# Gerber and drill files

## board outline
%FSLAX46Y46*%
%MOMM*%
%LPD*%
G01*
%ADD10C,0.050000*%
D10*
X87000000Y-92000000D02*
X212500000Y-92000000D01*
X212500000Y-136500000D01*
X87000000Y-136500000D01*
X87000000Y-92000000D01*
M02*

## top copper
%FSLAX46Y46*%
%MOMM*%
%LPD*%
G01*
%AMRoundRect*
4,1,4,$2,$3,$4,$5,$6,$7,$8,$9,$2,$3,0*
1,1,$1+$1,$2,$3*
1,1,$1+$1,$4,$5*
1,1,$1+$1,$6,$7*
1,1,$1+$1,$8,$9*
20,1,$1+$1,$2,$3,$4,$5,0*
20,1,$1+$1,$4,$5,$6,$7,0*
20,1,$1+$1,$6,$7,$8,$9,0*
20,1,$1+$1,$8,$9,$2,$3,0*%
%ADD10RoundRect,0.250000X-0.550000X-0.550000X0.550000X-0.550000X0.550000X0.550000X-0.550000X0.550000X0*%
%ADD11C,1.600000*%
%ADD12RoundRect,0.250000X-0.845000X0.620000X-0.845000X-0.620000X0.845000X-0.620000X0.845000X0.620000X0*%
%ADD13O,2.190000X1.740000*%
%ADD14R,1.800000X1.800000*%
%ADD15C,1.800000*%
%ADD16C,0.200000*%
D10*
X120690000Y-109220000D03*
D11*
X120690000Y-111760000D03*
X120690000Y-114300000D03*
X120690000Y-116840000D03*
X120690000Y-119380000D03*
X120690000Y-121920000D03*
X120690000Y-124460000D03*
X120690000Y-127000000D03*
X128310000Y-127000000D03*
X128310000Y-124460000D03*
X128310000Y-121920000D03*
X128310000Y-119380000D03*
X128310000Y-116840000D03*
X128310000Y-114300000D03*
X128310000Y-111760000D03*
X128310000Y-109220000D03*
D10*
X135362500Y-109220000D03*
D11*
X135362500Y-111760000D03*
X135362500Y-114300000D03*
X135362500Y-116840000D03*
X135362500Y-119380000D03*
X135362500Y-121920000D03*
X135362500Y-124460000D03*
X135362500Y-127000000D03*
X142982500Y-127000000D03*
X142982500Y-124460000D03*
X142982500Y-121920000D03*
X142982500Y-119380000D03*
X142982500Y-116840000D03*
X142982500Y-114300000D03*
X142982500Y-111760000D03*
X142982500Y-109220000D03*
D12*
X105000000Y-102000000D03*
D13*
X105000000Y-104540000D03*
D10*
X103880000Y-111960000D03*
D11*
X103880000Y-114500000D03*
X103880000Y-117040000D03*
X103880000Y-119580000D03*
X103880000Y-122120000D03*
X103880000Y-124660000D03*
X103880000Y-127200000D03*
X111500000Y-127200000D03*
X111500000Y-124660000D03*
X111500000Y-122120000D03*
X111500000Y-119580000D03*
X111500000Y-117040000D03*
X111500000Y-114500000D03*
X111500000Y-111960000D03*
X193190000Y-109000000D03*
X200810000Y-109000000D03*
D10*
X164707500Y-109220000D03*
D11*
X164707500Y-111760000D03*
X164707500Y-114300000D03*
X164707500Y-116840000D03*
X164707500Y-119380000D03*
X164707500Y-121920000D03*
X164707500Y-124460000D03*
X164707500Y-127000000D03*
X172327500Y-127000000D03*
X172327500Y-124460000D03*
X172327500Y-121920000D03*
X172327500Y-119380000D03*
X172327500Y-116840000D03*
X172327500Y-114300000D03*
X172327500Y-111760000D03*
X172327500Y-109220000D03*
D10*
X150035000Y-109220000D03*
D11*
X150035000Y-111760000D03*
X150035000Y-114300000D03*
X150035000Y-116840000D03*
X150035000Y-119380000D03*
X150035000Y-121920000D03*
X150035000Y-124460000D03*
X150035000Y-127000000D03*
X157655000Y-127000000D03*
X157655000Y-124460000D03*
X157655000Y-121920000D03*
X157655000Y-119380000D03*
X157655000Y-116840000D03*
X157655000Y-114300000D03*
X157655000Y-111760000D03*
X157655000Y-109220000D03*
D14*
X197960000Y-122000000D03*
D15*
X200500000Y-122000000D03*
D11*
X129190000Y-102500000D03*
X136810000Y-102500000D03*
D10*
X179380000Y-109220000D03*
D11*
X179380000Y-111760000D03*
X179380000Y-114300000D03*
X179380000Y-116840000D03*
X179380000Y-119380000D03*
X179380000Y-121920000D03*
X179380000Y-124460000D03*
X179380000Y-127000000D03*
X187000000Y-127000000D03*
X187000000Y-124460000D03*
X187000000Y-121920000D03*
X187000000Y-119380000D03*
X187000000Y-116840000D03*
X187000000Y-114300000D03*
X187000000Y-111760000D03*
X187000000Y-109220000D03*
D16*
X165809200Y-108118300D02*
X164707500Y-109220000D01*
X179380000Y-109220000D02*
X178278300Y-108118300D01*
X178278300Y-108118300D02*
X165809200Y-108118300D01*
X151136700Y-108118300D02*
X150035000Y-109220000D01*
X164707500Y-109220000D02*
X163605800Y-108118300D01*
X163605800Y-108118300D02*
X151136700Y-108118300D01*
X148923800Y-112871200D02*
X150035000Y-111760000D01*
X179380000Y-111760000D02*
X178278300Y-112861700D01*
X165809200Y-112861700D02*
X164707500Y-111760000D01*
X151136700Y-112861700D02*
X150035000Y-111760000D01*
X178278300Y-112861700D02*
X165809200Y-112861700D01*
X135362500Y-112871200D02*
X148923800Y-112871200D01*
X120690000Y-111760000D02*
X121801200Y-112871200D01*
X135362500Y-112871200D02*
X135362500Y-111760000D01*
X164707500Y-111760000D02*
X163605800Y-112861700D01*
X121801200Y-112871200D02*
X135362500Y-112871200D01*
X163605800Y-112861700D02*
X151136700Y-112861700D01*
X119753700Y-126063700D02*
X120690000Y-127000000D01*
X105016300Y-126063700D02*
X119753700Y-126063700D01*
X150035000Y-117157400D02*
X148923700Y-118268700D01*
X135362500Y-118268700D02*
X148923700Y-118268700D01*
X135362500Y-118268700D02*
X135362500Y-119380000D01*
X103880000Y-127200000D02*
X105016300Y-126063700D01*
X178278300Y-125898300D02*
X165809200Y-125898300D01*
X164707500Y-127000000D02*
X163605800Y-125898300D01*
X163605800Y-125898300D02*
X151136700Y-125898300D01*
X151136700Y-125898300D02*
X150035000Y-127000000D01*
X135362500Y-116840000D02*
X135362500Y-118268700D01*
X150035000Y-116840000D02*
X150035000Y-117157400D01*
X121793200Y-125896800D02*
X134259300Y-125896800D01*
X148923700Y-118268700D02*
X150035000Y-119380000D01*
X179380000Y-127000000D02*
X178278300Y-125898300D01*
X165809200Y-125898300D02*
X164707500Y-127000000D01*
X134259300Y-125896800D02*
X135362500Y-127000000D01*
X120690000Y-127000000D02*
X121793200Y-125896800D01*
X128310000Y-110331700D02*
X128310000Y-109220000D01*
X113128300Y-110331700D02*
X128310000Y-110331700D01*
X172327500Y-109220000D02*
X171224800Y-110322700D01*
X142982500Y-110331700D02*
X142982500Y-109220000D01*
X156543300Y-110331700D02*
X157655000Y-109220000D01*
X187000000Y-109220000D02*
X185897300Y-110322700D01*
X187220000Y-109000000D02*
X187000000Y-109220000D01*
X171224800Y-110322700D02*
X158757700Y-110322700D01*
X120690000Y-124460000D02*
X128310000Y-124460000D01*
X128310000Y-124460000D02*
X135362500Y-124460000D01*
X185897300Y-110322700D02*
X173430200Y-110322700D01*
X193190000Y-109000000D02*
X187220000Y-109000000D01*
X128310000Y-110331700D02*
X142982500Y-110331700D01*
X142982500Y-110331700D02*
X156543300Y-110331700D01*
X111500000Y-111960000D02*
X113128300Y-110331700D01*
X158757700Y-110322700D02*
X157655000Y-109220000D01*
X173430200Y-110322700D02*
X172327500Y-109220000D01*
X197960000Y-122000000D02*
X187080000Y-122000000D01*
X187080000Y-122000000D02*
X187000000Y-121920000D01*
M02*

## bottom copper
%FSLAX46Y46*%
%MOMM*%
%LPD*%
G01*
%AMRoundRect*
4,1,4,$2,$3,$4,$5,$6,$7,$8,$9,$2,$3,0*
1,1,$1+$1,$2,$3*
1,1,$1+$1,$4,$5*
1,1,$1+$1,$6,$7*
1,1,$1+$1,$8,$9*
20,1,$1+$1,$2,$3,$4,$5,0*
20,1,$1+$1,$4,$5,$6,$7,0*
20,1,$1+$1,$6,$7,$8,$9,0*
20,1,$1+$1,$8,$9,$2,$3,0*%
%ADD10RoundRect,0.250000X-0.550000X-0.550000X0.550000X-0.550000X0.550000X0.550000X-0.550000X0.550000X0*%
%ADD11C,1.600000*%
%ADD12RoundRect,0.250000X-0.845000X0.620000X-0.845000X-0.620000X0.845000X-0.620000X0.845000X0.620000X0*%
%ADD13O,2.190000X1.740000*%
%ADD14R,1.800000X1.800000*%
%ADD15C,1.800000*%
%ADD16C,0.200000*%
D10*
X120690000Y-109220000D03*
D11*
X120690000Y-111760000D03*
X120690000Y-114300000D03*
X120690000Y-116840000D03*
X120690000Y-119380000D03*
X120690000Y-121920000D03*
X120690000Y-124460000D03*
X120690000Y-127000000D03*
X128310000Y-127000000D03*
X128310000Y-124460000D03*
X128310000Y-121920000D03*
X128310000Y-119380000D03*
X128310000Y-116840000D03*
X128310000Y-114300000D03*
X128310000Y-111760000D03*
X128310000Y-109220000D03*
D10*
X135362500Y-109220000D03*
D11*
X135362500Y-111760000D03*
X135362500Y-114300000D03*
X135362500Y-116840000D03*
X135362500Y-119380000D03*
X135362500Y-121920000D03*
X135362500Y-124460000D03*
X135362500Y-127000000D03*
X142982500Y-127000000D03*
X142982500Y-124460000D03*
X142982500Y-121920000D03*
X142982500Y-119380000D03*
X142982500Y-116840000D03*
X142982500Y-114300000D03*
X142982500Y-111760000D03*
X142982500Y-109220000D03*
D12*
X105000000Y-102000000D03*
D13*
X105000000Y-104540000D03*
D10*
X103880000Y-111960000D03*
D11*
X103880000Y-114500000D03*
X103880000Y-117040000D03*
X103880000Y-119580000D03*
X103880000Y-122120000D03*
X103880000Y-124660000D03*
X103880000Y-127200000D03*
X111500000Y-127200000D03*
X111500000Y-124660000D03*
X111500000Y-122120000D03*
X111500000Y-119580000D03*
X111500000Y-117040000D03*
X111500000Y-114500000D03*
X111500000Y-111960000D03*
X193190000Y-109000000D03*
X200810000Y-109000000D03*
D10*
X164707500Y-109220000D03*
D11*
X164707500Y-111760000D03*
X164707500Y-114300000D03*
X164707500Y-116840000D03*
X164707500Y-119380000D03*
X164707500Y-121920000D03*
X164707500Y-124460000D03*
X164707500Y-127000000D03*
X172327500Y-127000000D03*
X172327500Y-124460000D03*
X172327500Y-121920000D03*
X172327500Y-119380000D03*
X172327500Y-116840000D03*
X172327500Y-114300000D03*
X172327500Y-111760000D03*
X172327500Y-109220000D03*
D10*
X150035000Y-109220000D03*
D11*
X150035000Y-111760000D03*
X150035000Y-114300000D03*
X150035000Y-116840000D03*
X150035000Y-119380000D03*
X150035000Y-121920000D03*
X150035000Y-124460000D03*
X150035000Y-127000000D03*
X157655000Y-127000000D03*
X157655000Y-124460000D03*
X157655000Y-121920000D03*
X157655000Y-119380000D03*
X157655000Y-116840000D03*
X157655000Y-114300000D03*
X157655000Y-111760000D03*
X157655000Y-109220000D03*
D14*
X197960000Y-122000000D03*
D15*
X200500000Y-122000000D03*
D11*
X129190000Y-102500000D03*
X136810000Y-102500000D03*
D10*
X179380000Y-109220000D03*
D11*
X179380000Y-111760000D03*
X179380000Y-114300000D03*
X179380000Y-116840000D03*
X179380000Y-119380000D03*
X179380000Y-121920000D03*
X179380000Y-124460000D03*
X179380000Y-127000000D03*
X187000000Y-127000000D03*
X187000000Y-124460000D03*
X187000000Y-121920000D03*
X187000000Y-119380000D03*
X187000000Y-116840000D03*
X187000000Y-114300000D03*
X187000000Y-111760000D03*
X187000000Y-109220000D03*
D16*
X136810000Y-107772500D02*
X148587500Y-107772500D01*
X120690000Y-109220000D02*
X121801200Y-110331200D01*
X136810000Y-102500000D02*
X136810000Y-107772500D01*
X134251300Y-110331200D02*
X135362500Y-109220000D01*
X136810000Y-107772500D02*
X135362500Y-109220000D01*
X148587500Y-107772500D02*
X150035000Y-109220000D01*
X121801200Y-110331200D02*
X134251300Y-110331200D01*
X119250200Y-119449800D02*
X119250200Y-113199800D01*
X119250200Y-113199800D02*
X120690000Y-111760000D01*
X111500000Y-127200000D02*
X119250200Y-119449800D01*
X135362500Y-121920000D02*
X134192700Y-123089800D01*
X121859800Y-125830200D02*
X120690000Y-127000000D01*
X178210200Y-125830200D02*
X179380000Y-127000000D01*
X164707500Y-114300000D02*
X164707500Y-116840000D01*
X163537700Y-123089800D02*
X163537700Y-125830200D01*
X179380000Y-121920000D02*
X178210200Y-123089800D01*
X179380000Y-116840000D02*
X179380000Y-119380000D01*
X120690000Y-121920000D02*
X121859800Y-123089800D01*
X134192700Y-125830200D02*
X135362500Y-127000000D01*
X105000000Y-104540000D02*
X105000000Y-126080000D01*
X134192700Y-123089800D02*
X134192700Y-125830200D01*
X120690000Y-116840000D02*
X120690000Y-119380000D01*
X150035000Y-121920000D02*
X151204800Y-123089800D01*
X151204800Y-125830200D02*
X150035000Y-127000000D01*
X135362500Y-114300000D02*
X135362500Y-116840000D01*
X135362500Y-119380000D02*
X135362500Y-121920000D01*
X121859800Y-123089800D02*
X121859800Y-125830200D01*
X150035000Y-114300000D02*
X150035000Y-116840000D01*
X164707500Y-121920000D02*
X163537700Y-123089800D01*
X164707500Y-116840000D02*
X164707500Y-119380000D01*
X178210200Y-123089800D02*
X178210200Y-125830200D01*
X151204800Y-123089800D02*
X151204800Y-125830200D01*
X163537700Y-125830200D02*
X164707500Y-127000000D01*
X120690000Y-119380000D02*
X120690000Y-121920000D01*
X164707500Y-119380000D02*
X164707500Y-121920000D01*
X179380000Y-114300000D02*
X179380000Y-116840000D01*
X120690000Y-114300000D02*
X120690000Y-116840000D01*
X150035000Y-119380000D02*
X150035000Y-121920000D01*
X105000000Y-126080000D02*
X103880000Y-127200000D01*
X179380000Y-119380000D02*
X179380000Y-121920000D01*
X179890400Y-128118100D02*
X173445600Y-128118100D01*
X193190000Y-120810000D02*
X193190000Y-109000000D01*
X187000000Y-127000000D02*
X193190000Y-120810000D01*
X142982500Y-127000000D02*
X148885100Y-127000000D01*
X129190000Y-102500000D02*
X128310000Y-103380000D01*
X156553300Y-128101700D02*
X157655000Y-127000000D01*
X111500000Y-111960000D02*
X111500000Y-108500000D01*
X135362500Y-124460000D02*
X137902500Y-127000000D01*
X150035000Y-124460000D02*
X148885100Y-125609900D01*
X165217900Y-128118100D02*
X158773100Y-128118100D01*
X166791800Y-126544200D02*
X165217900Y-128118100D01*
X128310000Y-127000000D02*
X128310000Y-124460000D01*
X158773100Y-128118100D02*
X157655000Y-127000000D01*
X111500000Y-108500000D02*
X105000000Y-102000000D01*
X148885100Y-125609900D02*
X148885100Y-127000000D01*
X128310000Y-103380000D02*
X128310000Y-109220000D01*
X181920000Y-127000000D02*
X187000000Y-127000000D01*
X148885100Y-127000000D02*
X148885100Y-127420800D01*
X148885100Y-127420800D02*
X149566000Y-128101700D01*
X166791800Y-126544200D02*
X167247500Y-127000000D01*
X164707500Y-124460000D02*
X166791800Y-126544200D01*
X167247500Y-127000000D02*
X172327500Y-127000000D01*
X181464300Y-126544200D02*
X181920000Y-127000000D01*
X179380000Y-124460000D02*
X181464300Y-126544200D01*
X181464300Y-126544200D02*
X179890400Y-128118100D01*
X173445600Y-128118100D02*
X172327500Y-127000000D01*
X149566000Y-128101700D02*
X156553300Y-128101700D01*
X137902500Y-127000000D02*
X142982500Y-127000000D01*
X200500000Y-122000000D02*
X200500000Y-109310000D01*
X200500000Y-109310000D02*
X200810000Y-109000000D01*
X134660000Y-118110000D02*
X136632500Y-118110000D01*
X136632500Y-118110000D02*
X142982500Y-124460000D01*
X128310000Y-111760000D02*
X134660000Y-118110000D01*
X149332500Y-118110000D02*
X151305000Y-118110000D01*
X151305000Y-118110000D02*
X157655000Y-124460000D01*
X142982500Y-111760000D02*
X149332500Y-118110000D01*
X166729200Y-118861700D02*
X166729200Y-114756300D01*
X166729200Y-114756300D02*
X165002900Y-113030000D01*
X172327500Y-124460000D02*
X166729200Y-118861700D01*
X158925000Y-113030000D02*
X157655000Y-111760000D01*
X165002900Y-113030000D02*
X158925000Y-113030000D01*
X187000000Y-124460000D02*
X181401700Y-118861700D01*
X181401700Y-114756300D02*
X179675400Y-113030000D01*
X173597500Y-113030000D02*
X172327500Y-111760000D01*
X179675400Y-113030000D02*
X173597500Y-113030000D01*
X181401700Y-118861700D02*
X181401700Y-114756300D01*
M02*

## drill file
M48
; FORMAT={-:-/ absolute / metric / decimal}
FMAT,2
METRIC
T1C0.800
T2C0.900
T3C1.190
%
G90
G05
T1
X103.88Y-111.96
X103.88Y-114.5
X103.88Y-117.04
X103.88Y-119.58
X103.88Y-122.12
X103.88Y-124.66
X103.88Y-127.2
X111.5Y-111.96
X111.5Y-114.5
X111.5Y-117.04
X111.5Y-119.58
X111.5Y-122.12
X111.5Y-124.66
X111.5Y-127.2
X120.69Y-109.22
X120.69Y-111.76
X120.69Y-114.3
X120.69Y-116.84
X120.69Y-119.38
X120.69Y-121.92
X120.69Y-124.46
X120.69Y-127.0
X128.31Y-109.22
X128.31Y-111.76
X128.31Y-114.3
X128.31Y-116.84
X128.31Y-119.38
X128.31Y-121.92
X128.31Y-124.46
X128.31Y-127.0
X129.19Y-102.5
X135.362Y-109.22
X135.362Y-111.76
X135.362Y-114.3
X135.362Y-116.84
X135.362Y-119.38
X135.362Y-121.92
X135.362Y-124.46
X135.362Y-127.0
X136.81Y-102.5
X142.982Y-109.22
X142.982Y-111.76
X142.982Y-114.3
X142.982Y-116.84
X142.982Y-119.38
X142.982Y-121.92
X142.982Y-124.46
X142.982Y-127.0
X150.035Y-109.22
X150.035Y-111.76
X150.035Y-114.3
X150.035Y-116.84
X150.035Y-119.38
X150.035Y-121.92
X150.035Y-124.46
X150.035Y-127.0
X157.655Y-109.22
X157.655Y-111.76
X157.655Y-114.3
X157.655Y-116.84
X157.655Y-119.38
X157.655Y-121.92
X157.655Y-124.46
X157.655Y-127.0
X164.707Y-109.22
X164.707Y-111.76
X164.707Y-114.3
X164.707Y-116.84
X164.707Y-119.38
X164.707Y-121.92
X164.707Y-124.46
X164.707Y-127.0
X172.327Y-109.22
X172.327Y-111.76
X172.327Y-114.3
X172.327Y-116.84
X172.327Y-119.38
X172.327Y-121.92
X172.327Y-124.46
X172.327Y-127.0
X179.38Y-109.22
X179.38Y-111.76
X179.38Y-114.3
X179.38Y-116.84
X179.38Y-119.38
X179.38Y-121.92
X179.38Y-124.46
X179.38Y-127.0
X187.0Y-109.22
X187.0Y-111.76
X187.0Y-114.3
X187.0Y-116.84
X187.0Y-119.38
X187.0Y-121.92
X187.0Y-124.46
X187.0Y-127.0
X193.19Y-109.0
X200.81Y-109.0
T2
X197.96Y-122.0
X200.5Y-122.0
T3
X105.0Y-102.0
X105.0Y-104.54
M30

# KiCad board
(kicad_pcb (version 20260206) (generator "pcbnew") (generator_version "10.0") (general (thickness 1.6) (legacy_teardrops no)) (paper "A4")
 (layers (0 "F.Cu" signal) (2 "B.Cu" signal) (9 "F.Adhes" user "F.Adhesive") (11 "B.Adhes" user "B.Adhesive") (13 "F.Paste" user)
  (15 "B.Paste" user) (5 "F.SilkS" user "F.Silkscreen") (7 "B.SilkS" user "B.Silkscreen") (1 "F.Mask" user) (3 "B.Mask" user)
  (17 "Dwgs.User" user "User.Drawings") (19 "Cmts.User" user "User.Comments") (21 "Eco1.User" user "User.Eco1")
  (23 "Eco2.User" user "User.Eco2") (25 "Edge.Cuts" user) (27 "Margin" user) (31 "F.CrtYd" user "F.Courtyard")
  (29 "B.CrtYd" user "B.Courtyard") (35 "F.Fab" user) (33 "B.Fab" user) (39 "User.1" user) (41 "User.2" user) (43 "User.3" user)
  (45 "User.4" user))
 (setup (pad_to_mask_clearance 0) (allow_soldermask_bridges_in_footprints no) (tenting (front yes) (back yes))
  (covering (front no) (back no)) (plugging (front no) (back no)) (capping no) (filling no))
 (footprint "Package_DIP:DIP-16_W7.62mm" (layer "F.Cu") (at 120.69 109.22)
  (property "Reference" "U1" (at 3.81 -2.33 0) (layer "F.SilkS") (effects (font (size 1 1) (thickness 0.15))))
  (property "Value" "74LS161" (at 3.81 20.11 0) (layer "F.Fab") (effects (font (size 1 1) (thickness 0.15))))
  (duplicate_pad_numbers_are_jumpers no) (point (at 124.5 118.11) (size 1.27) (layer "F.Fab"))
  (pad "1" thru_hole roundrect (at 0 0) (size 1.6 1.6) (drill 0.8) (layers "*.Cu" "*.Mask") (remove_unused_layers no)
   (roundrect_rratio 0.15625) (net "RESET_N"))
  (pad "2" thru_hole circle (at 0 2.54) (size 1.6 1.6) (drill 0.8) (layers "*.Cu" "*.Mask") (remove_unused_layers no) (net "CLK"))
  (pad "3" thru_hole circle (at 0 5.08) (size 1.6 1.6) (drill 0.8) (layers "*.Cu" "*.Mask") (remove_unused_layers no) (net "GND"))
  (pad "4" thru_hole circle (at 0 7.62) (size 1.6 1.6) (drill 0.8) (layers "*.Cu" "*.Mask") (remove_unused_layers no) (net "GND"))
  (pad "5" thru_hole circle (at 0 10.16) (size 1.6 1.6) (drill 0.8) (layers "*.Cu" "*.Mask") (remove_unused_layers no) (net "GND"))
  (pad "6" thru_hole circle (at 0 12.7) (size 1.6 1.6) (drill 0.8) (layers "*.Cu" "*.Mask") (remove_unused_layers no) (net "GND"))
  (pad "7" thru_hole circle (at 0 15.24) (size 1.6 1.6) (drill 0.8) (layers "*.Cu" "*.Mask") (remove_unused_layers no) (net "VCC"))
  (pad "8" thru_hole circle (at 0 17.78) (size 1.6 1.6) (drill 0.8) (layers "*.Cu" "*.Mask") (remove_unused_layers no) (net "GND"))
  (pad "9" thru_hole circle (at 7.62 17.78) (size 1.6 1.6) (drill 0.8) (layers "*.Cu" "*.Mask") (remove_unused_layers no) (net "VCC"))
  (pad "10" thru_hole circle (at 7.62 15.24) (size 1.6 1.6) (drill 0.8) (layers "*.Cu" "*.Mask") (remove_unused_layers no) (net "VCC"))
  (pad "11" thru_hole circle (at 7.62 12.7) (size 1.6 1.6) (drill 0.8) (layers "*.Cu" "*.Mask") (remove_unused_layers no))
  (pad "12" thru_hole circle (at 7.62 10.16) (size 1.6 1.6) (drill 0.8) (layers "*.Cu" "*.Mask") (remove_unused_layers no))
  (pad "13" thru_hole circle (at 7.62 7.62) (size 1.6 1.6) (drill 0.8) (layers "*.Cu" "*.Mask") (remove_unused_layers no))
  (pad "14" thru_hole circle (at 7.62 5.08) (size 1.6 1.6) (drill 0.8) (layers "*.Cu" "*.Mask") (remove_unused_layers no))
  (pad "15" thru_hole circle (at 7.62 2.54) (size 1.6 1.6) (drill 0.8) (layers "*.Cu" "*.Mask") (remove_unused_layers no) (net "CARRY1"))
  (pad "16" thru_hole circle (at 7.62 0) (size 1.6 1.6) (drill 0.8) (layers "*.Cu" "*.Mask") (remove_unused_layers no) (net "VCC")))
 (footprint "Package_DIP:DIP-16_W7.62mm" (layer "F.Cu") (at 135.3625 109.22)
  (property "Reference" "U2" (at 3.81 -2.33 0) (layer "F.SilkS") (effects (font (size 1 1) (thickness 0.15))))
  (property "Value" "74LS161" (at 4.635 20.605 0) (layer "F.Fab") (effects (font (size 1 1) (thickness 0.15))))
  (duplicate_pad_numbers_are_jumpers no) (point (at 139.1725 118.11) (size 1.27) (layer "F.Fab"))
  (pad "1" thru_hole roundrect (at 0 0) (size 1.6 1.6) (drill 0.8) (layers "*.Cu" "*.Mask") (remove_unused_layers no)
   (roundrect_rratio 0.15625) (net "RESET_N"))
  (pad "2" thru_hole circle (at 0 2.54) (size 1.6 1.6) (drill 0.8) (layers "*.Cu" "*.Mask") (remove_unused_layers no) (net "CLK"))
  (pad "3" thru_hole circle (at 0 5.08) (size 1.6 1.6) (drill 0.8) (layers "*.Cu" "*.Mask") (remove_unused_layers no) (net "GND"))
  (pad "4" thru_hole circle (at 0 7.62) (size 1.6 1.6) (drill 0.8) (layers "*.Cu" "*.Mask") (remove_unused_layers no) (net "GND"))
  (pad "5" thru_hole circle (at 0 10.16) (size 1.6 1.6) (drill 0.8) (layers "*.Cu" "*.Mask") (remove_unused_layers no) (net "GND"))
  (pad "6" thru_hole circle (at 0 12.7) (size 1.6 1.6) (drill 0.8) (layers "*.Cu" "*.Mask") (remove_unused_layers no) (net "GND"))
  (pad "7" thru_hole circle (at 0 15.24) (size 1.6 1.6) (drill 0.8) (layers "*.Cu" "*.Mask") (remove_unused_layers no) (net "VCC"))
  (pad "8" thru_hole circle (at 0 17.78) (size 1.6 1.6) (drill 0.8) (layers "*.Cu" "*.Mask") (remove_unused_layers no) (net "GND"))
  (pad "9" thru_hole circle (at 7.62 17.78) (size 1.6 1.6) (drill 0.8) (layers "*.Cu" "*.Mask") (remove_unused_layers no) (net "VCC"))
  (pad "10" thru_hole circle (at 7.62 15.24) (size 1.6 1.6) (drill 0.8) (layers "*.Cu" "*.Mask") (remove_unused_layers no) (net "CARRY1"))
  (pad "11" thru_hole circle (at 7.62 12.7) (size 1.6 1.6) (drill 0.8) (layers "*.Cu" "*.Mask") (remove_unused_layers no))
  (pad "12" thru_hole circle (at 7.62 10.16) (size 1.6 1.6) (drill 0.8) (layers "*.Cu" "*.Mask") (remove_unused_layers no))
  (pad "13" thru_hole circle (at 7.62 7.62) (size 1.6 1.6) (drill 0.8) (layers "*.Cu" "*.Mask") (remove_unused_layers no))
  (pad "14" thru_hole circle (at 7.62 5.08) (size 1.6 1.6) (drill 0.8) (layers "*.Cu" "*.Mask") (remove_unused_layers no))
  (pad "15" thru_hole circle (at 7.62 2.54) (size 1.6 1.6) (drill 0.8) (layers "*.Cu" "*.Mask") (remove_unused_layers no) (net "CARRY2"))
  (pad "16" thru_hole circle (at 7.62 0) (size 1.6 1.6) (drill 0.8) (layers "*.Cu" "*.Mask") (remove_unused_layers no) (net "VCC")))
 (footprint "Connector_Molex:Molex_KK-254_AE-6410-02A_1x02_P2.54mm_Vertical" (layer "F.Cu") (at 105 102 -90)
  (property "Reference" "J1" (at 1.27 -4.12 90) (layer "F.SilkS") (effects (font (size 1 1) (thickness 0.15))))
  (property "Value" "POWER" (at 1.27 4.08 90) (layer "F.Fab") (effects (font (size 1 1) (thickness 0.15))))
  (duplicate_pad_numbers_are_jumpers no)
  (pad "1" thru_hole roundrect (at 0 0 270) (size 1.74 2.19) (drill 1.19) (layers "*.Cu" "*.Mask") (remove_unused_layers no)
   (roundrect_rratio 0.143678) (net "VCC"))
  (pad "2" thru_hole oval (at 2.54 0 270) (size 1.74 2.19) (drill 1.19) (layers "*.Cu" "*.Mask") (remove_unused_layers no) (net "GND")))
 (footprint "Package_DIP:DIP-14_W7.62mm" (layer "F.Cu") (at 103.88 111.96)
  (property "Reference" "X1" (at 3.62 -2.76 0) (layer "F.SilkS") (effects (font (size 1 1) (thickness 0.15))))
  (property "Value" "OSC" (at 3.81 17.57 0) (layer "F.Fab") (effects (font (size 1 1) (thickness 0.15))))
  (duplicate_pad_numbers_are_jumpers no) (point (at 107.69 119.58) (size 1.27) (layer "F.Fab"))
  (pad "1" thru_hole roundrect (at 0 0) (size 1.6 1.6) (drill 0.8) (layers "*.Cu" "*.Mask") (remove_unused_layers no)
   (roundrect_rratio 0.15625))
  (pad "2" thru_hole circle (at 0 2.54) (size 1.6 1.6) (drill 0.8) (layers "*.Cu" "*.Mask") (remove_unused_layers no))
  (pad "3" thru_hole circle (at 0 5.08) (size 1.6 1.6) (drill 0.8) (layers "*.Cu" "*.Mask") (remove_unused_layers no))
  (pad "4" thru_hole circle (at 0 7.62) (size 1.6 1.6) (drill 0.8) (layers "*.Cu" "*.Mask") (remove_unused_layers no))
  (pad "5" thru_hole circle (at 0 10.16) (size 1.6 1.6) (drill 0.8) (layers "*.Cu" "*.Mask") (remove_unused_layers no))
  (pad "6" thru_hole circle (at 0 12.7) (size 1.6 1.6) (drill 0.8) (layers "*.Cu" "*.Mask") (remove_unused_layers no))
  (pad "7" thru_hole circle (at 0 15.24) (size 1.6 1.6) (drill 0.8) (layers "*.Cu" "*.Mask") (remove_unused_layers no) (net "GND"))
  (pad "8" thru_hole circle (at 7.62 15.24) (size 1.6 1.6) (drill 0.8) (layers "*.Cu" "*.Mask") (remove_unused_layers no) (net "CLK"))
  (pad "9" thru_hole circle (at 7.62 12.7) (size 1.6 1.6) (drill 0.8) (layers "*.Cu" "*.Mask") (remove_unused_layers no))
  (pad "10" thru_hole circle (at 7.62 10.16) (size 1.6 1.6) (drill 0.8) (layers "*.Cu" "*.Mask") (remove_unused_layers no))
  (pad "11" thru_hole circle (at 7.62 7.62) (size 1.6 1.6) (drill 0.8) (layers "*.Cu" "*.Mask") (remove_unused_layers no))
  (pad "12" thru_hole circle (at 7.62 5.08) (size 1.6 1.6) (drill 0.8) (layers "*.Cu" "*.Mask") (remove_unused_layers no))
  (pad "13" thru_hole circle (at 7.62 2.54) (size 1.6 1.6) (drill 0.8) (layers "*.Cu" "*.Mask") (remove_unused_layers no))
  (pad "14" thru_hole circle (at 7.62 0) (size 1.6 1.6) (drill 0.8) (layers "*.Cu" "*.Mask") (remove_unused_layers no) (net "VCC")))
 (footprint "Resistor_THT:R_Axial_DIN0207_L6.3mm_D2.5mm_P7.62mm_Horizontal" (layer "F.Cu") (at 193.19 109)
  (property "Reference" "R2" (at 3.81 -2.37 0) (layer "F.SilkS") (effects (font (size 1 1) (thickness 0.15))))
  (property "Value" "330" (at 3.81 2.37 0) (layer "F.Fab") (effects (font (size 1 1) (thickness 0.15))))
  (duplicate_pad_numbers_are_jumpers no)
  (pad "1" thru_hole circle (at 0 0) (size 1.6 1.6) (drill 0.8) (layers "*.Cu" "*.Mask") (remove_unused_layers no) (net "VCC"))
  (pad "2" thru_hole circle (at 7.62 0) (size 1.6 1.6) (drill 0.8) (layers "*.Cu" "*.Mask") (remove_unused_layers no) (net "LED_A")))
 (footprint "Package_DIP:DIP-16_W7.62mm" (layer "F.Cu") (at 164.7075 109.22)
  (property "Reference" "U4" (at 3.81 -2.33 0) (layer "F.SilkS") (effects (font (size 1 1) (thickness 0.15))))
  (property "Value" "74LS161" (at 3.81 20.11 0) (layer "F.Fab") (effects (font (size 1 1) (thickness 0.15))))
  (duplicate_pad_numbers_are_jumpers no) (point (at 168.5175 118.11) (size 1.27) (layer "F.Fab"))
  (pad "1" thru_hole roundrect (at 0 0) (size 1.6 1.6) (drill 0.8) (layers "*.Cu" "*.Mask") (remove_unused_layers no)
   (roundrect_rratio 0.15625) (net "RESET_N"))
  (pad "2" thru_hole circle (at 0 2.54) (size 1.6 1.6) (drill 0.8) (layers "*.Cu" "*.Mask") (remove_unused_layers no) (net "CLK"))
  (pad "3" thru_hole circle (at 0 5.08) (size 1.6 1.6) (drill 0.8) (layers "*.Cu" "*.Mask") (remove_unused_layers no) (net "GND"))
  (pad "4" thru_hole circle (at 0 7.62) (size 1.6 1.6) (drill 0.8) (layers "*.Cu" "*.Mask") (remove_unused_layers no) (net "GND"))
  (pad "5" thru_hole circle (at 0 10.16) (size 1.6 1.6) (drill 0.8) (layers "*.Cu" "*.Mask") (remove_unused_layers no) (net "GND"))
  (pad "6" thru_hole circle (at 0 12.7) (size 1.6 1.6) (drill 0.8) (layers "*.Cu" "*.Mask") (remove_unused_layers no) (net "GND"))
  (pad "7" thru_hole circle (at 0 15.24) (size 1.6 1.6) (drill 0.8) (layers "*.Cu" "*.Mask") (remove_unused_layers no) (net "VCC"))
  (pad "8" thru_hole circle (at 0 17.78) (size 1.6 1.6) (drill 0.8) (layers "*.Cu" "*.Mask") (remove_unused_layers no) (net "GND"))
  (pad "9" thru_hole circle (at 7.62 17.78) (size 1.6 1.6) (drill 0.8) (layers "*.Cu" "*.Mask") (remove_unused_layers no) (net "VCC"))
  (pad "10" thru_hole circle (at 7.62 15.24) (size 1.6 1.6) (drill 0.8) (layers "*.Cu" "*.Mask") (remove_unused_layers no) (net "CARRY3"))
  (pad "11" thru_hole circle (at 7.62 12.7) (size 1.6 1.6) (drill 0.8) (layers "*.Cu" "*.Mask") (remove_unused_layers no))
  (pad "12" thru_hole circle (at 7.62 10.16) (size 1.6 1.6) (drill 0.8) (layers "*.Cu" "*.Mask") (remove_unused_layers no))
  (pad "13" thru_hole circle (at 7.62 7.62) (size 1.6 1.6) (drill 0.8) (layers "*.Cu" "*.Mask") (remove_unused_layers no))
  (pad "14" thru_hole circle (at 7.62 5.08) (size 1.6 1.6) (drill 0.8) (layers "*.Cu" "*.Mask") (remove_unused_layers no))
  (pad "15" thru_hole circle (at 7.62 2.54) (size 1.6 1.6) (drill 0.8) (layers "*.Cu" "*.Mask") (remove_unused_layers no) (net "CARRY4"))
  (pad "16" thru_hole circle (at 7.62 0) (size 1.6 1.6) (drill 0.8) (layers "*.Cu" "*.Mask") (remove_unused_layers no) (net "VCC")))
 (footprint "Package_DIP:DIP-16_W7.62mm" (layer "F.Cu") (at 150.035 109.22)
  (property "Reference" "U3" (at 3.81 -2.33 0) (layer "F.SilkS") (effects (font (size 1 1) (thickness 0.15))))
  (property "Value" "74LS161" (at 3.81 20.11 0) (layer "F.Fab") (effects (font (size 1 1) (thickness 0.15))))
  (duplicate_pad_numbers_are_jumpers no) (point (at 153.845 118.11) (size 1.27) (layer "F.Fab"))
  (pad "1" thru_hole roundrect (at 0 0) (size 1.6 1.6) (drill 0.8) (layers "*.Cu" "*.Mask") (remove_unused_layers no)
   (roundrect_rratio 0.15625) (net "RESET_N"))
  (pad "2" thru_hole circle (at 0 2.54) (size 1.6 1.6) (drill 0.8) (layers "*.Cu" "*.Mask") (remove_unused_layers no) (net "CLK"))
  (pad "3" thru_hole circle (at 0 5.08) (size 1.6 1.6) (drill 0.8) (layers "*.Cu" "*.Mask") (remove_unused_layers no) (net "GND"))
  (pad "4" thru_hole circle (at 0 7.62) (size 1.6 1.6) (drill 0.8) (layers "*.Cu" "*.Mask") (remove_unused_layers no) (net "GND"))
  (pad "5" thru_hole circle (at 0 10.16) (size 1.6 1.6) (drill 0.8) (layers "*.Cu" "*.Mask") (remove_unused_layers no) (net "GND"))
  (pad "6" thru_hole circle (at 0 12.7) (size 1.6 1.6) (drill 0.8) (layers "*.Cu" "*.Mask") (remove_unused_layers no) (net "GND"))
  (pad "7" thru_hole circle (at 0 15.24) (size 1.6 1.6) (drill 0.8) (layers "*.Cu" "*.Mask") (remove_unused_layers no) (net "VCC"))
  (pad "8" thru_hole circle (at 0 17.78) (size 1.6 1.6) (drill 0.8) (layers "*.Cu" "*.Mask") (remove_unused_layers no) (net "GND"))
  (pad "9" thru_hole circle (at 7.62 17.78) (size 1.6 1.6) (drill 0.8) (layers "*.Cu" "*.Mask") (remove_unused_layers no) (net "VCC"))
  (pad "10" thru_hole circle (at 7.62 15.24) (size 1.6 1.6) (drill 0.8) (layers "*.Cu" "*.Mask") (remove_unused_layers no) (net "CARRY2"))
  (pad "11" thru_hole circle (at 7.62 12.7) (size 1.6 1.6) (drill 0.8) (layers "*.Cu" "*.Mask") (remove_unused_layers no))
  (pad "12" thru_hole circle (at 7.62 10.16) (size 1.6 1.6) (drill 0.8) (layers "*.Cu" "*.Mask") (remove_unused_layers no))
  (pad "13" thru_hole circle (at 7.62 7.62) (size 1.6 1.6) (drill 0.8) (layers "*.Cu" "*.Mask") (remove_unused_layers no))
  (pad "14" thru_hole circle (at 7.62 5.08) (size 1.6 1.6) (drill 0.8) (layers "*.Cu" "*.Mask") (remove_unused_layers no))
  (pad "15" thru_hole circle (at 7.62 2.54) (size 1.6 1.6) (drill 0.8) (layers "*.Cu" "*.Mask") (remove_unused_layers no) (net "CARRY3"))
  (pad "16" thru_hole circle (at 7.62 0) (size 1.6 1.6) (drill 0.8) (layers "*.Cu" "*.Mask") (remove_unused_layers no) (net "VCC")))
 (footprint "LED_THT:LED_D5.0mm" (layer "F.Cu") (at 197.96 122)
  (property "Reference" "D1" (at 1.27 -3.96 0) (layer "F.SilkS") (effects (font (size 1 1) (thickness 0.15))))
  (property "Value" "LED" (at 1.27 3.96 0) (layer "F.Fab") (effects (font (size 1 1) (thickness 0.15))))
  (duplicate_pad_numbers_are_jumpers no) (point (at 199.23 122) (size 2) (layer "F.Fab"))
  (pad "1" thru_hole rect (at 0 0) (size 1.8 1.8) (drill 0.9) (layers "*.Cu" "*.Mask") (remove_unused_layers no) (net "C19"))
  (pad "2" thru_hole circle (at 2.54 0) (size 1.8 1.8) (drill 0.9) (layers "*.Cu" "*.Mask") (remove_unused_layers no) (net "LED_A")))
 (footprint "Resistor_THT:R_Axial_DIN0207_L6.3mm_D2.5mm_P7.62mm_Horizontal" (layer "F.Cu") (at 129.19 102.5)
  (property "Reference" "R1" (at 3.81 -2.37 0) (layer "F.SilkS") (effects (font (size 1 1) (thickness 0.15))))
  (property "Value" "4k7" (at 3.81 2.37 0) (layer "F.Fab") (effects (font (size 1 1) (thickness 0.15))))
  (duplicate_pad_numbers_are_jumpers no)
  (pad "1" thru_hole circle (at 0 0) (size 1.6 1.6) (drill 0.8) (layers "*.Cu" "*.Mask") (remove_unused_layers no) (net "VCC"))
  (pad "2" thru_hole circle (at 7.62 0) (size 1.6 1.6) (drill 0.8) (layers "*.Cu" "*.Mask") (remove_unused_layers no) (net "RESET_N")))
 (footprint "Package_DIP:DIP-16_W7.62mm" (layer "F.Cu") (at 179.38 109.22)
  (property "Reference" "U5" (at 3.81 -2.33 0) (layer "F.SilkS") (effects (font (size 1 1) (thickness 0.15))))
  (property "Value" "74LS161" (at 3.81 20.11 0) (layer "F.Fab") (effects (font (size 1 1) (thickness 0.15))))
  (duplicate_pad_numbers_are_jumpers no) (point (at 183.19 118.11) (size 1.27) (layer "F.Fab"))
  (pad "1" thru_hole roundrect (at 0 0) (size 1.6 1.6) (drill 0.8) (layers "*.Cu" "*.Mask") (remove_unused_layers no)
   (roundrect_rratio 0.15625) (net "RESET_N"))
  (pad "2" thru_hole circle (at 0 2.54) (size 1.6 1.6) (drill 0.8) (layers "*.Cu" "*.Mask") (remove_unused_layers no) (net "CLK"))
  (pad "3" thru_hole circle (at 0 5.08) (size 1.6 1.6) (drill 0.8) (layers "*.Cu" "*.Mask") (remove_unused_layers no) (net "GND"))
  (pad "4" thru_hole circle (at 0 7.62) (size 1.6 1.6) (drill 0.8) (layers "*.Cu" "*.Mask") (remove_unused_layers no) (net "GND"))
  (pad "5" thru_hole circle (at 0 10.16) (size 1.6 1.6) (drill 0.8) (layers "*.Cu" "*.Mask") (remove_unused_layers no) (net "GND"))
  (pad "6" thru_hole circle (at 0 12.7) (size 1.6 1.6) (drill 0.8) (layers "*.Cu" "*.Mask") (remove_unused_layers no) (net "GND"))
  (pad "7" thru_hole circle (at 0 15.24) (size 1.6 1.6) (drill 0.8) (layers "*.Cu" "*.Mask") (remove_unused_layers no) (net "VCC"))
  (pad "8" thru_hole circle (at 0 17.78) (size 1.6 1.6) (drill 0.8) (layers "*.Cu" "*.Mask") (remove_unused_layers no) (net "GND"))
  (pad "9" thru_hole circle (at 7.62 17.78) (size 1.6 1.6) (drill 0.8) (layers "*.Cu" "*.Mask") (remove_unused_layers no) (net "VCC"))
  (pad "10" thru_hole circle (at 7.62 15.24) (size 1.6 1.6) (drill 0.8) (layers "*.Cu" "*.Mask") (remove_unused_layers no) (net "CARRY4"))
  (pad "11" thru_hole circle (at 7.62 12.7) (size 1.6 1.6) (drill 0.8) (layers "*.Cu" "*.Mask") (remove_unused_layers no) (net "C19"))
  (pad "12" thru_hole circle (at 7.62 10.16) (size 1.6 1.6) (drill 0.8) (layers "*.Cu" "*.Mask") (remove_unused_layers no))
  (pad "13" thru_hole circle (at 7.62 7.62) (size 1.6 1.6) (drill 0.8) (layers "*.Cu" "*.Mask") (remove_unused_layers no))
  (pad "14" thru_hole circle (at 7.62 5.08) (size 1.6 1.6) (drill 0.8) (layers "*.Cu" "*.Mask") (remove_unused_layers no))
  (pad "15" thru_hole circle (at 7.62 2.54) (size 1.6 1.6) (drill 0.8) (layers "*.Cu" "*.Mask") (remove_unused_layers no))
  (pad "16" thru_hole circle (at 7.62 0) (size 1.6 1.6) (drill 0.8) (layers "*.Cu" "*.Mask") (remove_unused_layers no) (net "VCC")))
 (gr_rect (start 87 92) (end 212.5 136.5) (stroke (width 0.05) (type default)) (fill no) (layer "Edge.Cuts"))
 (segment (start 165.8092 108.1183) (end 164.7075 109.22) (width 0.2) (layer "F.Cu") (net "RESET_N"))
 (segment (start 179.38 109.22) (end 178.2783 108.1183) (width 0.2) (layer "F.Cu") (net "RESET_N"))
 (segment (start 178.2783 108.1183) (end 165.8092 108.1183) (width 0.2) (layer "F.Cu") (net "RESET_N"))
 (segment (start 151.1367 108.1183) (end 150.035 109.22) (width 0.2) (layer "F.Cu") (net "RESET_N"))
 (segment (start 164.7075 109.22) (end 163.6058 108.1183) (width 0.2) (layer "F.Cu") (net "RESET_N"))
 (segment (start 163.6058 108.1183) (end 151.1367 108.1183) (width 0.2) (layer "F.Cu") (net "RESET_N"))
 (segment (start 136.81 107.7725) (end 148.5875 107.7725) (width 0.2) (layer "B.Cu") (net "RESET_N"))
 (segment (start 120.69 109.22) (end 121.8012 110.3312) (width 0.2) (layer "B.Cu") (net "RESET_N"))
 (segment (start 136.81 102.5) (end 136.81 107.7725) (width 0.2) (layer "B.Cu") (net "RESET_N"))
 (segment (start 134.2513 110.3312) (end 135.3625 109.22) (width 0.2) (layer "B.Cu") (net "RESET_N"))
 (segment (start 136.81 107.7725) (end 135.3625 109.22) (width 0.2) (layer "B.Cu") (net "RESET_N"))
 (segment (start 148.5875 107.7725) (end 150.035 109.22) (width 0.2) (layer "B.Cu") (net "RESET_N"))
 (segment (start 121.8012 110.3312) (end 134.2513 110.3312) (width 0.2) (layer "B.Cu") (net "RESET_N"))
 (segment (start 148.9238 112.8712) (end 150.035 111.76) (width 0.2) (layer "F.Cu") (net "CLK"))
 (segment (start 179.38 111.76) (end 178.2783 112.8617) (width 0.2) (layer "F.Cu") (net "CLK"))
 (segment (start 165.8092 112.8617) (end 164.7075 111.76) (width 0.2) (layer "F.Cu") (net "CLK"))
 (segment (start 151.1367 112.8617) (end 150.035 111.76) (width 0.2) (layer "F.Cu") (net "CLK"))
 (segment (start 178.2783 112.8617) (end 165.8092 112.8617) (width 0.2) (layer "F.Cu") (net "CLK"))
 (segment (start 135.3625 112.8712) (end 148.9238 112.8712) (width 0.2) (layer "F.Cu") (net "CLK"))
 (segment (start 120.69 111.76) (end 121.8012 112.8712) (width 0.2) (layer "F.Cu") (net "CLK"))
 (segment (start 135.3625 112.8712) (end 135.3625 111.76) (width 0.2) (layer "F.Cu") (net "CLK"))
 (segment (start 164.7075 111.76) (end 163.6058 112.8617) (width 0.2) (layer "F.Cu") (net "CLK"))
 (segment (start 121.8012 112.8712) (end 135.3625 112.8712) (width 0.2) (layer "F.Cu") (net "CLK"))
 (segment (start 163.6058 112.8617) (end 151.1367 112.8617) (width 0.2) (layer "F.Cu") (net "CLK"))
 (segment (start 119.2502 119.4498) (end 119.2502 113.1998) (width 0.2) (layer "B.Cu") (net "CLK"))
 (segment (start 119.2502 113.1998) (end 120.69 111.76) (width 0.2) (layer "B.Cu") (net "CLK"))
 (segment (start 111.5 127.2) (end 119.2502 119.4498) (width 0.2) (layer "B.Cu") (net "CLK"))
 (segment (start 119.7537 126.0637) (end 120.69 127) (width 0.2) (layer "F.Cu") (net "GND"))
 (segment (start 105.0163 126.0637) (end 119.7537 126.0637) (width 0.2) (layer "F.Cu") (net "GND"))
 (segment (start 150.035 117.1574) (end 148.9237 118.2687) (width 0.2) (layer "F.Cu") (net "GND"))
 (segment (start 135.3625 118.2687) (end 148.9237 118.2687) (width 0.2) (layer "F.Cu") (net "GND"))
 (segment (start 135.3625 118.2687) (end 135.3625 119.38) (width 0.2) (layer "F.Cu") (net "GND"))
 (segment (start 103.88 127.2) (end 105.0163 126.0637) (width 0.2) (layer "F.Cu") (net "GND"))
 (segment (start 178.2783 125.8983) (end 165.8092 125.8983) (width 0.2) (layer "F.Cu") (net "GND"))
 (segment (start 164.7075 127) (end 163.6058 125.8983) (width 0.2) (layer "F.Cu") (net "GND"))
 (segment (start 163.6058 125.8983) (end 151.1367 125.8983) (width 0.2) (layer "F.Cu") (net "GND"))
 (segment (start 151.1367 125.8983) (end 150.035 127) (width 0.2) (layer "F.Cu") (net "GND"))
 (segment (start 135.3625 116.84) (end 135.3625 118.2687) (width 0.2) (layer "F.Cu") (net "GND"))
 (segment (start 150.035 116.84) (end 150.035 117.1574) (width 0.2) (layer "F.Cu") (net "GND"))
 (segment (start 121.7932 125.8968) (end 134.2593 125.8968) (width 0.2) (layer "F.Cu") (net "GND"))
 (segment (start 148.9237 118.2687) (end 150.035 119.38) (width 0.2) (layer "F.Cu") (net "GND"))
 (segment (start 179.38 127) (end 178.2783 125.8983) (width 0.2) (layer "F.Cu") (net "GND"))
 (segment (start 165.8092 125.8983) (end 164.7075 127) (width 0.2) (layer "F.Cu") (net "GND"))
 (segment (start 134.2593 125.8968) (end 135.3625 127) (width 0.2) (layer "F.Cu") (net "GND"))
 (segment (start 120.69 127) (end 121.7932 125.8968) (width 0.2) (layer "F.Cu") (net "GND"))
 (segment (start 135.3625 121.92) (end 134.1927 123.0898) (width 0.2) (layer "B.Cu") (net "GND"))
 (segment (start 121.8598 125.8302) (end 120.69 127) (width 0.2) (layer "B.Cu") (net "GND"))
 (segment (start 178.2102 125.8302) (end 179.38 127) (width 0.2) (layer "B.Cu") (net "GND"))
 (segment (start 164.7075 114.3) (end 164.7075 116.84) (width 0.2) (layer "B.Cu") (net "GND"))
 (segment (start 163.5377 123.0898) (end 163.5377 125.8302) (width 0.2) (layer "B.Cu") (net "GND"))
 (segment (start 179.38 121.92) (end 178.2102 123.0898) (width 0.2) (layer "B.Cu") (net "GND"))
 (segment (start 179.38 116.84) (end 179.38 119.38) (width 0.2) (layer "B.Cu") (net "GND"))
 (segment (start 120.69 121.92) (end 121.8598 123.0898) (width 0.2) (layer "B.Cu") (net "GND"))
 (segment (start 134.1927 125.8302) (end 135.3625 127) (width 0.2) (layer "B.Cu") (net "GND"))
 (segment (start 105 104.54) (end 105 126.08) (width 0.2) (layer "B.Cu") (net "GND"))
 (segment (start 134.1927 123.0898) (end 134.1927 125.8302) (width 0.2) (layer "B.Cu") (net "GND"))
 (segment (start 120.69 116.84) (end 120.69 119.38) (width 0.2) (layer "B.Cu") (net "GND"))
 (segment (start 150.035 121.92) (end 151.2048 123.0898) (width 0.2) (layer "B.Cu") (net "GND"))
 (segment (start 151.2048 125.8302) (end 150.035 127) (width 0.2) (layer "B.Cu") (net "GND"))
 (segment (start 135.3625 114.3) (end 135.3625 116.84) (width 0.2) (layer "B.Cu") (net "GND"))
 (segment (start 135.3625 119.38) (end 135.3625 121.92) (width 0.2) (layer "B.Cu") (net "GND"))
 (segment (start 121.8598 123.0898) (end 121.8598 125.8302) (width 0.2) (layer "B.Cu") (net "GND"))
 (segment (start 150.035 114.3) (end 150.035 116.84) (width 0.2) (layer "B.Cu") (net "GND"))
 (segment (start 164.7075 121.92) (end 163.5377 123.0898) (width 0.2) (layer "B.Cu") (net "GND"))
 (segment (start 164.7075 116.84) (end 164.7075 119.38) (width 0.2) (layer "B.Cu") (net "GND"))
 (segment (start 178.2102 123.0898) (end 178.2102 125.8302) (width 0.2) (layer "B.Cu") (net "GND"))
 (segment (start 151.2048 123.0898) (end 151.2048 125.8302) (width 0.2) (layer "B.Cu") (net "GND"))
 (segment (start 163.5377 125.8302) (end 164.7075 127) (width 0.2) (layer "B.Cu") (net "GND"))
 (segment (start 120.69 119.38) (end 120.69 121.92) (width 0.2) (layer "B.Cu") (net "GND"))
 (segment (start 164.7075 119.38) (end 164.7075 121.92) (width 0.2) (layer "B.Cu") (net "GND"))
 (segment (start 179.38 114.3) (end 179.38 116.84) (width 0.2) (layer "B.Cu") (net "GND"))
 (segment (start 120.69 114.3) (end 120.69 116.84) (width 0.2) (layer "B.Cu") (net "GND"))
 (segment (start 150.035 119.38) (end 150.035 121.92) (width 0.2) (layer "B.Cu") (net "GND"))
 (segment (start 105 126.08) (end 103.88 127.2) (width 0.2) (layer "B.Cu") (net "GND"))
 (segment (start 179.38 119.38) (end 179.38 121.92) (width 0.2) (layer "B.Cu") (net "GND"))
 (segment (start 128.31 110.3317) (end 128.31 109.22) (width 0.2) (layer "F.Cu") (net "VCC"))
 (segment (start 113.1283 110.3317) (end 128.31 110.3317) (width 0.2) (layer "F.Cu") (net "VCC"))
 (segment (start 172.3275 109.22) (end 171.2248 110.3227) (width 0.2) (layer "F.Cu") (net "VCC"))
 (segment (start 142.9825 110.3317) (end 142.9825 109.22) (width 0.2) (layer "F.Cu") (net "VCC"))
 (segment (start 156.5433 110.3317) (end 157.655 109.22) (width 0.2) (layer "F.Cu") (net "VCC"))
 (segment (start 187 109.22) (end 185.8973 110.3227) (width 0.2) (layer "F.Cu") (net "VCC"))
 (segment (start 187.22 109) (end 187 109.22) (width 0.2) (layer "F.Cu") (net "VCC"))
 (segment (start 171.2248 110.3227) (end 158.7577 110.3227) (width 0.2) (layer "F.Cu") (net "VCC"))
 (segment (start 120.69 124.46) (end 128.31 124.46) (width 0.2) (layer "F.Cu") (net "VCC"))
 (segment (start 128.31 124.46) (end 135.3625 124.46) (width 0.2) (layer "F.Cu") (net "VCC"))
 (segment (start 185.8973 110.3227) (end 173.4302 110.3227) (width 0.2) (layer "F.Cu") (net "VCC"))
 (segment (start 193.19 109) (end 187.22 109) (width 0.2) (layer "F.Cu") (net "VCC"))
 (segment (start 128.31 110.3317) (end 142.9825 110.3317) (width 0.2) (layer "F.Cu") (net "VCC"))
 (segment (start 142.9825 110.3317) (end 156.5433 110.3317) (width 0.2) (layer "F.Cu") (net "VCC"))
 (segment (start 111.5 111.96) (end 113.1283 110.3317) (width 0.2) (layer "F.Cu") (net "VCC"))
 (segment (start 158.7577 110.3227) (end 157.655 109.22) (width 0.2) (layer "F.Cu") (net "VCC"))
 (segment (start 173.4302 110.3227) (end 172.3275 109.22) (width 0.2) (layer "F.Cu") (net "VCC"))
 (segment (start 179.8904 128.1181) (end 173.4456 128.1181) (width 0.2) (layer "B.Cu") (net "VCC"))
 (segment (start 193.19 120.81) (end 193.19 109) (width 0.2) (layer "B.Cu") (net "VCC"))
 (segment (start 187 127) (end 193.19 120.81) (width 0.2) (layer "B.Cu") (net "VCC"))
 (segment (start 142.9825 127) (end 148.8851 127) (width 0.2) (layer "B.Cu") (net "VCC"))
 (segment (start 129.19 102.5) (end 128.31 103.38) (width 0.2) (layer "B.Cu") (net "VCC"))
 (segment (start 156.5533 128.1017) (end 157.655 127) (width 0.2) (layer "B.Cu") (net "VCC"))
 (segment (start 111.5 111.96) (end 111.5 108.5) (width 0.2) (layer "B.Cu") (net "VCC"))
 (segment (start 135.3625 124.46) (end 137.9025 127) (width 0.2) (layer "B.Cu") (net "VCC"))
 (segment (start 150.035 124.46) (end 148.8851 125.6099) (width 0.2) (layer "B.Cu") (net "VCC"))
 (segment (start 165.2179 128.1181) (end 158.7731 128.1181) (width 0.2) (layer "B.Cu") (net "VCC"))
 (segment (start 166.7918 126.5442) (end 165.2179 128.1181) (width 0.2) (layer "B.Cu") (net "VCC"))
 (segment (start 128.31 127) (end 128.31 124.46) (width 0.2) (layer "B.Cu") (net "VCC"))
 (segment (start 158.7731 128.1181) (end 157.655 127) (width 0.2) (layer "B.Cu") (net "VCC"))
 (segment (start 111.5 108.5) (end 105 102) (width 0.2) (layer "B.Cu") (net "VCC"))
 (segment (start 148.8851 125.6099) (end 148.8851 127) (width 0.2) (layer "B.Cu") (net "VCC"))
 (segment (start 128.31 103.38) (end 128.31 109.22) (width 0.2) (layer "B.Cu") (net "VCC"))
 (segment (start 181.92 127) (end 187 127) (width 0.2) (layer "B.Cu") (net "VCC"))
 (segment (start 148.8851 127) (end 148.8851 127.4208) (width 0.2) (layer "B.Cu") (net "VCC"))
 (segment (start 148.8851 127.4208) (end 149.566 128.1017) (width 0.2) (layer "B.Cu") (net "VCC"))
 (segment (start 166.7918 126.5442) (end 167.2475 127) (width 0.2) (layer "B.Cu") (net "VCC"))
 (segment (start 164.7075 124.46) (end 166.7918 126.5442) (width 0.2) (layer "B.Cu") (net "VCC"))
 (segment (start 167.2475 127) (end 172.3275 127) (width 0.2) (layer "B.Cu") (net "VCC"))
 (segment (start 181.4643 126.5442) (end 181.92 127) (width 0.2) (layer "B.Cu") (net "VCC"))
 (segment (start 179.38 124.46) (end 181.4643 126.5442) (width 0.2) (layer "B.Cu") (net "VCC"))
 (segment (start 181.4643 126.5442) (end 179.8904 128.1181) (width 0.2) (layer "B.Cu") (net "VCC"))
 (segment (start 173.4456 128.1181) (end 172.3275 127) (width 0.2) (layer "B.Cu") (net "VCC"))
 (segment (start 149.566 128.1017) (end 156.5533 128.1017) (width 0.2) (layer "B.Cu") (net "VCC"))
 (segment (start 137.9025 127) (end 142.9825 127) (width 0.2) (layer "B.Cu") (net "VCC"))
 (segment (start 200.5 122) (end 200.5 109.31) (width 0.2) (layer "B.Cu") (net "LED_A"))
 (segment (start 200.5 109.31) (end 200.81 109) (width 0.2) (layer "B.Cu") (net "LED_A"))
 (segment (start 134.66 118.11) (end 136.6325 118.11) (width 0.2) (layer "B.Cu") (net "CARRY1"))
 (segment (start 136.6325 118.11) (end 142.9825 124.46) (width 0.2) (layer "B.Cu") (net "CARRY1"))
 (segment (start 128.31 111.76) (end 134.66 118.11) (width 0.2) (layer "B.Cu") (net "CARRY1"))
 (segment (start 149.3325 118.11) (end 151.305 118.11) (width 0.2) (layer "B.Cu") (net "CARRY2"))
 (segment (start 151.305 118.11) (end 157.655 124.46) (width 0.2) (layer "B.Cu") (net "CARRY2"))
 (segment (start 142.9825 111.76) (end 149.3325 118.11) (width 0.2) (layer "B.Cu") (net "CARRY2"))
 (segment (start 166.7292 118.8617) (end 166.7292 114.7563) (width 0.2) (layer "B.Cu") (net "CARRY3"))
 (segment (start 166.7292 114.7563) (end 165.0029 113.03) (width 0.2) (layer "B.Cu") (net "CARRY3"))
 (segment (start 172.3275 124.46) (end 166.7292 118.8617) (width 0.2) (layer "B.Cu") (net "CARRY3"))
 (segment (start 158.925 113.03) (end 157.655 111.76) (width 0.2) (layer "B.Cu") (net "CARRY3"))
 (segment (start 165.0029 113.03) (end 158.925 113.03) (width 0.2) (layer "B.Cu") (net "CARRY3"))
 (segment (start 187 124.46) (end 181.4017 118.8617) (width 0.2) (layer "B.Cu") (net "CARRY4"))
 (segment (start 181.4017 114.7563) (end 179.6754 113.03) (width 0.2) (layer "B.Cu") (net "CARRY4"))
 (segment (start 173.5975 113.03) (end 172.3275 111.76) (width 0.2) (layer "B.Cu") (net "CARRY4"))
 (segment (start 179.6754 113.03) (end 173.5975 113.03) (width 0.2) (layer "B.Cu") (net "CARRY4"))
 (segment (start 181.4017 118.8617) (end 181.4017 114.7563) (width 0.2) (layer "B.Cu") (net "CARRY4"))
 (segment (start 197.96 122) (end 187.08 122) (width 0.2) (layer "F.Cu") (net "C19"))
 (segment (start 187.08 122) (end 187 121.92) (width 0.2) (layer "F.Cu") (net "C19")))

